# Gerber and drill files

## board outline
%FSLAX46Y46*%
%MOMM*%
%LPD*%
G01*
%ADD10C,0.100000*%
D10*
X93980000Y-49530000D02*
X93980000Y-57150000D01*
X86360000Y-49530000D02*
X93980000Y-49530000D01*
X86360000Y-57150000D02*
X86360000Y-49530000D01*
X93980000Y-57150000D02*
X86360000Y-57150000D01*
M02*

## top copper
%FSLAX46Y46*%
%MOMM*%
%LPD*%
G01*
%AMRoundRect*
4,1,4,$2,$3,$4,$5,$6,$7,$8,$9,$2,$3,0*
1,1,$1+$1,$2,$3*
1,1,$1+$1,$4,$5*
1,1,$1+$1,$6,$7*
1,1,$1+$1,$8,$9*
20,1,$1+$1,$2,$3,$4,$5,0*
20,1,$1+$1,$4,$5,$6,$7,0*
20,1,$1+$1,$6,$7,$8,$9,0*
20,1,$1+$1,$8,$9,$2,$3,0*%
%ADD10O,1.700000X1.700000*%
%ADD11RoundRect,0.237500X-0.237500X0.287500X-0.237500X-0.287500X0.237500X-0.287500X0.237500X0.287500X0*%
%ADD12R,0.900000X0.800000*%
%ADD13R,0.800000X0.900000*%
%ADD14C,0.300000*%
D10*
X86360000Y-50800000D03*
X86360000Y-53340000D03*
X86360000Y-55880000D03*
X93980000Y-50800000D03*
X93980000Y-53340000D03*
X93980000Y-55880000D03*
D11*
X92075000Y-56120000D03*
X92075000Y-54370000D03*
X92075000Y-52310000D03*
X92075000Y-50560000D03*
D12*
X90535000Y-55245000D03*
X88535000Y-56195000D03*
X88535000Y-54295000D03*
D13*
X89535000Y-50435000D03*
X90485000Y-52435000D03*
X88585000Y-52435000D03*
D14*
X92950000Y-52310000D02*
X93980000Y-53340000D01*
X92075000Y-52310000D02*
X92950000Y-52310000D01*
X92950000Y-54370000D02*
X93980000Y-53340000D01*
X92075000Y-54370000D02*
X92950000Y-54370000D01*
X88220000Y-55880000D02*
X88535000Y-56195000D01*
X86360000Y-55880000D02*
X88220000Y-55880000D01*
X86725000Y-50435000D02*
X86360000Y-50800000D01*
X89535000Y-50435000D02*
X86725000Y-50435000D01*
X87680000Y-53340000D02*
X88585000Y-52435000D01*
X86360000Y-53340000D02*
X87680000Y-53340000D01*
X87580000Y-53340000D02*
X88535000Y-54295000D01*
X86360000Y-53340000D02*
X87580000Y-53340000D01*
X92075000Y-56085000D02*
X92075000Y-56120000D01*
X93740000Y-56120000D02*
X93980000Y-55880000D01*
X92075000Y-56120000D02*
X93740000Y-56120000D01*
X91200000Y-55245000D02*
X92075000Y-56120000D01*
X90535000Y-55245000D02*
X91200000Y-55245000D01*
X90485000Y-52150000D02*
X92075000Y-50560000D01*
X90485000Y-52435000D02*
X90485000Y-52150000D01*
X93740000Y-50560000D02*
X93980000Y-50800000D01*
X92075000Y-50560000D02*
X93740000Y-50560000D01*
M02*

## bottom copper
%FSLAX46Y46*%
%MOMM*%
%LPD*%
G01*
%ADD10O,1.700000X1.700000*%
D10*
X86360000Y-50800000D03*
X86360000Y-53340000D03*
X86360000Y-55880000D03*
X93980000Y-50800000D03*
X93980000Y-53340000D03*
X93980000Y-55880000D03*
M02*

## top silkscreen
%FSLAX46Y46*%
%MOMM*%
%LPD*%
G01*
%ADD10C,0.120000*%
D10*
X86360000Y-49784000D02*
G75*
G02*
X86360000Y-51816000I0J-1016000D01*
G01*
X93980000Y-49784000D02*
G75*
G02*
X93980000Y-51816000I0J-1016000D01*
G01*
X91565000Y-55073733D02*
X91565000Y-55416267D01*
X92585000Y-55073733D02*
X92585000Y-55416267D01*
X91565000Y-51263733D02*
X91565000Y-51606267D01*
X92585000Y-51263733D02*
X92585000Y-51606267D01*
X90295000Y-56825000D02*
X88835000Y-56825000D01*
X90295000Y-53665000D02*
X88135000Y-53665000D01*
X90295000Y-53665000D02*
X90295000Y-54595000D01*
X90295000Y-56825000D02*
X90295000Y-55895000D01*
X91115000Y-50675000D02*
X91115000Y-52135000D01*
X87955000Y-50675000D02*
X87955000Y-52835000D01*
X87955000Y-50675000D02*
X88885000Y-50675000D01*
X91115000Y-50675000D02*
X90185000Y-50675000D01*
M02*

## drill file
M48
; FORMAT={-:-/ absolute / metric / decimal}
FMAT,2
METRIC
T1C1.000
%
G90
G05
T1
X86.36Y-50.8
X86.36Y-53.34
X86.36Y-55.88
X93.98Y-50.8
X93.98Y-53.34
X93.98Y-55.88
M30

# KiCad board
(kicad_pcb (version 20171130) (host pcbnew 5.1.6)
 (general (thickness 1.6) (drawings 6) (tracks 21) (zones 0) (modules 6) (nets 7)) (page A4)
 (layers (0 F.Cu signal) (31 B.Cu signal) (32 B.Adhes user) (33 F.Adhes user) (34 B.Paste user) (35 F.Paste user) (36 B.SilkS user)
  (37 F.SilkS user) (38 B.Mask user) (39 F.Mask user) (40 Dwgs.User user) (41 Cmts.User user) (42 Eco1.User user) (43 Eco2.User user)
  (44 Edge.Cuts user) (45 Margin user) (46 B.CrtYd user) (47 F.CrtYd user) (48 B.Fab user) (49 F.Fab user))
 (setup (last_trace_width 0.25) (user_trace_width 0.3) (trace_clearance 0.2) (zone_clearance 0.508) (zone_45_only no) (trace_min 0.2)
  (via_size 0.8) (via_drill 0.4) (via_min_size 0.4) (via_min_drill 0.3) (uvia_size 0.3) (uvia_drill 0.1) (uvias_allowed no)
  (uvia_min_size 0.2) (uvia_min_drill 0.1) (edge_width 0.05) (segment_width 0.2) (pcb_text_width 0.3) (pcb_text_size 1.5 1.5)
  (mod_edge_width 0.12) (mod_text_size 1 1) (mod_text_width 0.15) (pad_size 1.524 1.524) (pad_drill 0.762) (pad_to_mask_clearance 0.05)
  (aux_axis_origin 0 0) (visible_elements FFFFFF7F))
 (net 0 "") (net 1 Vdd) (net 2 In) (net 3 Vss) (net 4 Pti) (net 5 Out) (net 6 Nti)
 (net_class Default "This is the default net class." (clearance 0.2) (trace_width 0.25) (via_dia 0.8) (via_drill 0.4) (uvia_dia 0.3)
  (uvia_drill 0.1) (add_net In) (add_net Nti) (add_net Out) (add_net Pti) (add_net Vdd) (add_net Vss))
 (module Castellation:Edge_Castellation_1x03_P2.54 (layer F.Cu) (at 86.36 50.8)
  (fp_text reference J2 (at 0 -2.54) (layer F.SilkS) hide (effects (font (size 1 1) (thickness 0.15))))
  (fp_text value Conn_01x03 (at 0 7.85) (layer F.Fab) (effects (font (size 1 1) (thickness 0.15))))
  (fp_arc (start 0 0) (end 0 1.016) (angle -180) (layer F.SilkS) (width 0.12))
  (pad 1 thru_hole oval (at 0 0) (size 1.7 1.7) (drill 1) (layers *.Cu *.Mask) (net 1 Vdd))
  (pad 2 thru_hole oval (at 0 2.54) (size 1.7 1.7) (drill 1) (layers *.Cu *.Mask) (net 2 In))
  (pad 3 thru_hole oval (at 0 5.08) (size 1.7 1.7) (drill 1) (layers *.Cu *.Mask) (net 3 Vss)))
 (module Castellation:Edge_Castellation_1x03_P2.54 (layer F.Cu) (at 93.98 50.8)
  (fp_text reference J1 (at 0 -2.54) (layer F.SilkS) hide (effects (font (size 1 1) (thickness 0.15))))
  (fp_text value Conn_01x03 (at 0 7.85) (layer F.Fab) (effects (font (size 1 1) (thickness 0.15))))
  (fp_arc (start 0 0) (end 0 1.016) (angle -180) (layer F.SilkS) (width 0.12))
  (pad 1 thru_hole oval (at 0 0) (size 1.7 1.7) (drill 1) (layers *.Cu *.Mask) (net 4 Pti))
  (pad 2 thru_hole oval (at 0 2.54) (size 1.7 1.7) (drill 1) (layers *.Cu *.Mask) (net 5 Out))
  (pad 3 thru_hole oval (at 0 5.08) (size 1.7 1.7) (drill 1) (layers *.Cu *.Mask) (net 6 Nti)))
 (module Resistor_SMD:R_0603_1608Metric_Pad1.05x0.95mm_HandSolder (layer F.Cu) (at 92.075 55.245 270)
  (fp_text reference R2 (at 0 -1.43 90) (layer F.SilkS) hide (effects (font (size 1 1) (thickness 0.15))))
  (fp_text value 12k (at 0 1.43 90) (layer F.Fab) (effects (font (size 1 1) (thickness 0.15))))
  (fp_line (start -0.171267 0.51) (end 0.171267 0.51) (layer F.SilkS) (width 0.12))
  (fp_line (start -0.171267 -0.51) (end 0.171267 -0.51) (layer F.SilkS) (width 0.12))
  (pad 2 smd roundrect (at 0.875 0 270) (size 1.05 0.95) (layers F.Cu F.Paste F.Mask) (roundrect_rratio 0.25) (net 6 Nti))
  (pad 1 smd roundrect (at -0.875 0 270) (size 1.05 0.95) (layers F.Cu F.Paste F.Mask) (roundrect_rratio 0.25) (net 5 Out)))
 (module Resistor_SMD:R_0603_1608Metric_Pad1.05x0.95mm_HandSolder (layer F.Cu) (at 92.075 51.435 270)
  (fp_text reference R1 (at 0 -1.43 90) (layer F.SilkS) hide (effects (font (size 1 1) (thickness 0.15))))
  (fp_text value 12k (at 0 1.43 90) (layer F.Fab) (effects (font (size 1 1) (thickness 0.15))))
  (fp_line (start -0.171267 0.51) (end 0.171267 0.51) (layer F.SilkS) (width 0.12))
  (fp_line (start -0.171267 -0.51) (end 0.171267 -0.51) (layer F.SilkS) (width 0.12))
  (pad 2 smd roundrect (at 0.875 0 270) (size 1.05 0.95) (layers F.Cu F.Paste F.Mask) (roundrect_rratio 0.25) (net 5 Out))
  (pad 1 smd roundrect (at -0.875 0 270) (size 1.05 0.95) (layers F.Cu F.Paste F.Mask) (roundrect_rratio 0.25) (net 4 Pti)))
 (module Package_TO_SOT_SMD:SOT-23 (layer F.Cu) (at 89.535 55.245)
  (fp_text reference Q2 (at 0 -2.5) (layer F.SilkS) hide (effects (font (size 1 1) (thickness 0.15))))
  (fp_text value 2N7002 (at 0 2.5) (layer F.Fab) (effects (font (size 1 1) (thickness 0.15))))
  (fp_line (start 0.76 1.58) (end -0.7 1.58) (layer F.SilkS) (width 0.12))
  (fp_line (start 0.76 -1.58) (end -1.4 -1.58) (layer F.SilkS) (width 0.12))
  (fp_line (start 0.76 -1.58) (end 0.76 -0.65) (layer F.SilkS) (width 0.12))
  (fp_line (start 0.76 1.58) (end 0.76 0.65) (layer F.SilkS) (width 0.12))
  (pad 3 smd rect (at 1 0) (size 0.9 0.8) (layers F.Cu F.Paste F.Mask) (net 6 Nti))
  (pad 2 smd rect (at -1 0.95) (size 0.9 0.8) (layers F.Cu F.Paste F.Mask) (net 3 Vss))
  (pad 1 smd rect (at -1 -0.95) (size 0.9 0.8) (layers F.Cu F.Paste F.Mask) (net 2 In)))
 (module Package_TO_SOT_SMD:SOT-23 (layer F.Cu) (at 89.535 51.435 90)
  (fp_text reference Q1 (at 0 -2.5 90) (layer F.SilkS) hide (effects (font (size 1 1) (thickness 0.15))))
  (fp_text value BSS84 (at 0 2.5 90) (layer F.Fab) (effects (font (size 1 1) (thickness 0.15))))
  (fp_line (start 0.76 1.58) (end -0.7 1.58) (layer F.SilkS) (width 0.12))
  (fp_line (start 0.76 -1.58) (end -1.4 -1.58) (layer F.SilkS) (width 0.12))
  (fp_line (start 0.76 -1.58) (end 0.76 -0.65) (layer F.SilkS) (width 0.12))
  (fp_line (start 0.76 1.58) (end 0.76 0.65) (layer F.SilkS) (width 0.12))
  (pad 3 smd rect (at 1 0 90) (size 0.9 0.8) (layers F.Cu F.Paste F.Mask) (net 1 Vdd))
  (pad 2 smd rect (at -1 0.95 90) (size 0.9 0.8) (layers F.Cu F.Paste F.Mask) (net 4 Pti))
  (pad 1 smd rect (at -1 -0.95 90) (size 0.9 0.8) (layers F.Cu F.Paste F.Mask) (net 2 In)))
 (gr_line (start 93.98 49.53) (end 93.98 57.15) (layer Edge.Cuts) (width 0.1))
 (gr_line (start 86.36 49.53) (end 93.98 49.53) (layer Edge.Cuts) (width 0.1))
 (gr_line (start 86.36 57.15) (end 86.36 49.53) (layer Edge.Cuts) (width 0.1))
 (gr_line (start 93.98 57.15) (end 86.36 57.15) (layer Edge.Cuts) (width 0.1))
 (segment (start 92.95 52.31) (end 93.98 53.34) (width 0.3) (layer F.Cu) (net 5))
 (segment (start 92.075 52.31) (end 92.95 52.31) (width 0.3) (layer F.Cu) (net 5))
 (segment (start 92.95 54.37) (end 93.98 53.34) (width 0.3) (layer F.Cu) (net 5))
 (segment (start 92.075 54.37) (end 92.95 54.37) (width 0.3) (layer F.Cu) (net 5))
 (segment (start 88.22 55.88) (end 88.535 56.195) (width 0.3) (layer F.Cu) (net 3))
 (segment (start 86.36 55.88) (end 88.22 55.88) (width 0.3) (layer F.Cu) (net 3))
 (segment (start 86.725 50.435) (end 86.36 50.8) (width 0.3) (layer F.Cu) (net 1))
 (segment (start 89.535 50.435) (end 86.725 50.435) (width 0.3) (layer F.Cu) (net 1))
 (segment (start 87.68 53.34) (end 88.585 52.435) (width 0.3) (layer F.Cu) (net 2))
 (segment (start 86.36 53.34) (end 87.68 53.34) (width 0.3) (layer F.Cu) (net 2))
 (segment (start 87.58 53.34) (end 88.535 54.295) (width 0.3) (layer F.Cu) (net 2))
 (segment (start 86.36 53.34) (end 87.58 53.34) (width 0.3) (layer F.Cu) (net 2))
 (segment (start 92.075 56.085) (end 92.075 56.12) (width 0.3) (layer F.Cu) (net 6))
 (segment (start 93.74 56.12) (end 93.98 55.88) (width 0.3) (layer F.Cu) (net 6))
 (segment (start 92.075 56.12) (end 93.74 56.12) (width 0.3) (layer F.Cu) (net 6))
 (segment (start 91.2 55.245) (end 92.075 56.12) (width 0.3) (layer F.Cu) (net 6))
 (segment (start 90.535 55.245) (end 91.2 55.245) (width 0.3) (layer F.Cu) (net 6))
 (segment (start 90.485 52.15) (end 92.075 50.56) (width 0.3) (layer F.Cu) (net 4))
 (segment (start 90.485 52.435) (end 90.485 52.15) (width 0.3) (layer F.Cu) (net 4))
 (segment (start 93.74 50.56) (end 93.98 50.8) (width 0.3) (layer F.Cu) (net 4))
 (segment (start 92.075 50.56) (end 93.74 50.56) (width 0.3) (layer F.Cu) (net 4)))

